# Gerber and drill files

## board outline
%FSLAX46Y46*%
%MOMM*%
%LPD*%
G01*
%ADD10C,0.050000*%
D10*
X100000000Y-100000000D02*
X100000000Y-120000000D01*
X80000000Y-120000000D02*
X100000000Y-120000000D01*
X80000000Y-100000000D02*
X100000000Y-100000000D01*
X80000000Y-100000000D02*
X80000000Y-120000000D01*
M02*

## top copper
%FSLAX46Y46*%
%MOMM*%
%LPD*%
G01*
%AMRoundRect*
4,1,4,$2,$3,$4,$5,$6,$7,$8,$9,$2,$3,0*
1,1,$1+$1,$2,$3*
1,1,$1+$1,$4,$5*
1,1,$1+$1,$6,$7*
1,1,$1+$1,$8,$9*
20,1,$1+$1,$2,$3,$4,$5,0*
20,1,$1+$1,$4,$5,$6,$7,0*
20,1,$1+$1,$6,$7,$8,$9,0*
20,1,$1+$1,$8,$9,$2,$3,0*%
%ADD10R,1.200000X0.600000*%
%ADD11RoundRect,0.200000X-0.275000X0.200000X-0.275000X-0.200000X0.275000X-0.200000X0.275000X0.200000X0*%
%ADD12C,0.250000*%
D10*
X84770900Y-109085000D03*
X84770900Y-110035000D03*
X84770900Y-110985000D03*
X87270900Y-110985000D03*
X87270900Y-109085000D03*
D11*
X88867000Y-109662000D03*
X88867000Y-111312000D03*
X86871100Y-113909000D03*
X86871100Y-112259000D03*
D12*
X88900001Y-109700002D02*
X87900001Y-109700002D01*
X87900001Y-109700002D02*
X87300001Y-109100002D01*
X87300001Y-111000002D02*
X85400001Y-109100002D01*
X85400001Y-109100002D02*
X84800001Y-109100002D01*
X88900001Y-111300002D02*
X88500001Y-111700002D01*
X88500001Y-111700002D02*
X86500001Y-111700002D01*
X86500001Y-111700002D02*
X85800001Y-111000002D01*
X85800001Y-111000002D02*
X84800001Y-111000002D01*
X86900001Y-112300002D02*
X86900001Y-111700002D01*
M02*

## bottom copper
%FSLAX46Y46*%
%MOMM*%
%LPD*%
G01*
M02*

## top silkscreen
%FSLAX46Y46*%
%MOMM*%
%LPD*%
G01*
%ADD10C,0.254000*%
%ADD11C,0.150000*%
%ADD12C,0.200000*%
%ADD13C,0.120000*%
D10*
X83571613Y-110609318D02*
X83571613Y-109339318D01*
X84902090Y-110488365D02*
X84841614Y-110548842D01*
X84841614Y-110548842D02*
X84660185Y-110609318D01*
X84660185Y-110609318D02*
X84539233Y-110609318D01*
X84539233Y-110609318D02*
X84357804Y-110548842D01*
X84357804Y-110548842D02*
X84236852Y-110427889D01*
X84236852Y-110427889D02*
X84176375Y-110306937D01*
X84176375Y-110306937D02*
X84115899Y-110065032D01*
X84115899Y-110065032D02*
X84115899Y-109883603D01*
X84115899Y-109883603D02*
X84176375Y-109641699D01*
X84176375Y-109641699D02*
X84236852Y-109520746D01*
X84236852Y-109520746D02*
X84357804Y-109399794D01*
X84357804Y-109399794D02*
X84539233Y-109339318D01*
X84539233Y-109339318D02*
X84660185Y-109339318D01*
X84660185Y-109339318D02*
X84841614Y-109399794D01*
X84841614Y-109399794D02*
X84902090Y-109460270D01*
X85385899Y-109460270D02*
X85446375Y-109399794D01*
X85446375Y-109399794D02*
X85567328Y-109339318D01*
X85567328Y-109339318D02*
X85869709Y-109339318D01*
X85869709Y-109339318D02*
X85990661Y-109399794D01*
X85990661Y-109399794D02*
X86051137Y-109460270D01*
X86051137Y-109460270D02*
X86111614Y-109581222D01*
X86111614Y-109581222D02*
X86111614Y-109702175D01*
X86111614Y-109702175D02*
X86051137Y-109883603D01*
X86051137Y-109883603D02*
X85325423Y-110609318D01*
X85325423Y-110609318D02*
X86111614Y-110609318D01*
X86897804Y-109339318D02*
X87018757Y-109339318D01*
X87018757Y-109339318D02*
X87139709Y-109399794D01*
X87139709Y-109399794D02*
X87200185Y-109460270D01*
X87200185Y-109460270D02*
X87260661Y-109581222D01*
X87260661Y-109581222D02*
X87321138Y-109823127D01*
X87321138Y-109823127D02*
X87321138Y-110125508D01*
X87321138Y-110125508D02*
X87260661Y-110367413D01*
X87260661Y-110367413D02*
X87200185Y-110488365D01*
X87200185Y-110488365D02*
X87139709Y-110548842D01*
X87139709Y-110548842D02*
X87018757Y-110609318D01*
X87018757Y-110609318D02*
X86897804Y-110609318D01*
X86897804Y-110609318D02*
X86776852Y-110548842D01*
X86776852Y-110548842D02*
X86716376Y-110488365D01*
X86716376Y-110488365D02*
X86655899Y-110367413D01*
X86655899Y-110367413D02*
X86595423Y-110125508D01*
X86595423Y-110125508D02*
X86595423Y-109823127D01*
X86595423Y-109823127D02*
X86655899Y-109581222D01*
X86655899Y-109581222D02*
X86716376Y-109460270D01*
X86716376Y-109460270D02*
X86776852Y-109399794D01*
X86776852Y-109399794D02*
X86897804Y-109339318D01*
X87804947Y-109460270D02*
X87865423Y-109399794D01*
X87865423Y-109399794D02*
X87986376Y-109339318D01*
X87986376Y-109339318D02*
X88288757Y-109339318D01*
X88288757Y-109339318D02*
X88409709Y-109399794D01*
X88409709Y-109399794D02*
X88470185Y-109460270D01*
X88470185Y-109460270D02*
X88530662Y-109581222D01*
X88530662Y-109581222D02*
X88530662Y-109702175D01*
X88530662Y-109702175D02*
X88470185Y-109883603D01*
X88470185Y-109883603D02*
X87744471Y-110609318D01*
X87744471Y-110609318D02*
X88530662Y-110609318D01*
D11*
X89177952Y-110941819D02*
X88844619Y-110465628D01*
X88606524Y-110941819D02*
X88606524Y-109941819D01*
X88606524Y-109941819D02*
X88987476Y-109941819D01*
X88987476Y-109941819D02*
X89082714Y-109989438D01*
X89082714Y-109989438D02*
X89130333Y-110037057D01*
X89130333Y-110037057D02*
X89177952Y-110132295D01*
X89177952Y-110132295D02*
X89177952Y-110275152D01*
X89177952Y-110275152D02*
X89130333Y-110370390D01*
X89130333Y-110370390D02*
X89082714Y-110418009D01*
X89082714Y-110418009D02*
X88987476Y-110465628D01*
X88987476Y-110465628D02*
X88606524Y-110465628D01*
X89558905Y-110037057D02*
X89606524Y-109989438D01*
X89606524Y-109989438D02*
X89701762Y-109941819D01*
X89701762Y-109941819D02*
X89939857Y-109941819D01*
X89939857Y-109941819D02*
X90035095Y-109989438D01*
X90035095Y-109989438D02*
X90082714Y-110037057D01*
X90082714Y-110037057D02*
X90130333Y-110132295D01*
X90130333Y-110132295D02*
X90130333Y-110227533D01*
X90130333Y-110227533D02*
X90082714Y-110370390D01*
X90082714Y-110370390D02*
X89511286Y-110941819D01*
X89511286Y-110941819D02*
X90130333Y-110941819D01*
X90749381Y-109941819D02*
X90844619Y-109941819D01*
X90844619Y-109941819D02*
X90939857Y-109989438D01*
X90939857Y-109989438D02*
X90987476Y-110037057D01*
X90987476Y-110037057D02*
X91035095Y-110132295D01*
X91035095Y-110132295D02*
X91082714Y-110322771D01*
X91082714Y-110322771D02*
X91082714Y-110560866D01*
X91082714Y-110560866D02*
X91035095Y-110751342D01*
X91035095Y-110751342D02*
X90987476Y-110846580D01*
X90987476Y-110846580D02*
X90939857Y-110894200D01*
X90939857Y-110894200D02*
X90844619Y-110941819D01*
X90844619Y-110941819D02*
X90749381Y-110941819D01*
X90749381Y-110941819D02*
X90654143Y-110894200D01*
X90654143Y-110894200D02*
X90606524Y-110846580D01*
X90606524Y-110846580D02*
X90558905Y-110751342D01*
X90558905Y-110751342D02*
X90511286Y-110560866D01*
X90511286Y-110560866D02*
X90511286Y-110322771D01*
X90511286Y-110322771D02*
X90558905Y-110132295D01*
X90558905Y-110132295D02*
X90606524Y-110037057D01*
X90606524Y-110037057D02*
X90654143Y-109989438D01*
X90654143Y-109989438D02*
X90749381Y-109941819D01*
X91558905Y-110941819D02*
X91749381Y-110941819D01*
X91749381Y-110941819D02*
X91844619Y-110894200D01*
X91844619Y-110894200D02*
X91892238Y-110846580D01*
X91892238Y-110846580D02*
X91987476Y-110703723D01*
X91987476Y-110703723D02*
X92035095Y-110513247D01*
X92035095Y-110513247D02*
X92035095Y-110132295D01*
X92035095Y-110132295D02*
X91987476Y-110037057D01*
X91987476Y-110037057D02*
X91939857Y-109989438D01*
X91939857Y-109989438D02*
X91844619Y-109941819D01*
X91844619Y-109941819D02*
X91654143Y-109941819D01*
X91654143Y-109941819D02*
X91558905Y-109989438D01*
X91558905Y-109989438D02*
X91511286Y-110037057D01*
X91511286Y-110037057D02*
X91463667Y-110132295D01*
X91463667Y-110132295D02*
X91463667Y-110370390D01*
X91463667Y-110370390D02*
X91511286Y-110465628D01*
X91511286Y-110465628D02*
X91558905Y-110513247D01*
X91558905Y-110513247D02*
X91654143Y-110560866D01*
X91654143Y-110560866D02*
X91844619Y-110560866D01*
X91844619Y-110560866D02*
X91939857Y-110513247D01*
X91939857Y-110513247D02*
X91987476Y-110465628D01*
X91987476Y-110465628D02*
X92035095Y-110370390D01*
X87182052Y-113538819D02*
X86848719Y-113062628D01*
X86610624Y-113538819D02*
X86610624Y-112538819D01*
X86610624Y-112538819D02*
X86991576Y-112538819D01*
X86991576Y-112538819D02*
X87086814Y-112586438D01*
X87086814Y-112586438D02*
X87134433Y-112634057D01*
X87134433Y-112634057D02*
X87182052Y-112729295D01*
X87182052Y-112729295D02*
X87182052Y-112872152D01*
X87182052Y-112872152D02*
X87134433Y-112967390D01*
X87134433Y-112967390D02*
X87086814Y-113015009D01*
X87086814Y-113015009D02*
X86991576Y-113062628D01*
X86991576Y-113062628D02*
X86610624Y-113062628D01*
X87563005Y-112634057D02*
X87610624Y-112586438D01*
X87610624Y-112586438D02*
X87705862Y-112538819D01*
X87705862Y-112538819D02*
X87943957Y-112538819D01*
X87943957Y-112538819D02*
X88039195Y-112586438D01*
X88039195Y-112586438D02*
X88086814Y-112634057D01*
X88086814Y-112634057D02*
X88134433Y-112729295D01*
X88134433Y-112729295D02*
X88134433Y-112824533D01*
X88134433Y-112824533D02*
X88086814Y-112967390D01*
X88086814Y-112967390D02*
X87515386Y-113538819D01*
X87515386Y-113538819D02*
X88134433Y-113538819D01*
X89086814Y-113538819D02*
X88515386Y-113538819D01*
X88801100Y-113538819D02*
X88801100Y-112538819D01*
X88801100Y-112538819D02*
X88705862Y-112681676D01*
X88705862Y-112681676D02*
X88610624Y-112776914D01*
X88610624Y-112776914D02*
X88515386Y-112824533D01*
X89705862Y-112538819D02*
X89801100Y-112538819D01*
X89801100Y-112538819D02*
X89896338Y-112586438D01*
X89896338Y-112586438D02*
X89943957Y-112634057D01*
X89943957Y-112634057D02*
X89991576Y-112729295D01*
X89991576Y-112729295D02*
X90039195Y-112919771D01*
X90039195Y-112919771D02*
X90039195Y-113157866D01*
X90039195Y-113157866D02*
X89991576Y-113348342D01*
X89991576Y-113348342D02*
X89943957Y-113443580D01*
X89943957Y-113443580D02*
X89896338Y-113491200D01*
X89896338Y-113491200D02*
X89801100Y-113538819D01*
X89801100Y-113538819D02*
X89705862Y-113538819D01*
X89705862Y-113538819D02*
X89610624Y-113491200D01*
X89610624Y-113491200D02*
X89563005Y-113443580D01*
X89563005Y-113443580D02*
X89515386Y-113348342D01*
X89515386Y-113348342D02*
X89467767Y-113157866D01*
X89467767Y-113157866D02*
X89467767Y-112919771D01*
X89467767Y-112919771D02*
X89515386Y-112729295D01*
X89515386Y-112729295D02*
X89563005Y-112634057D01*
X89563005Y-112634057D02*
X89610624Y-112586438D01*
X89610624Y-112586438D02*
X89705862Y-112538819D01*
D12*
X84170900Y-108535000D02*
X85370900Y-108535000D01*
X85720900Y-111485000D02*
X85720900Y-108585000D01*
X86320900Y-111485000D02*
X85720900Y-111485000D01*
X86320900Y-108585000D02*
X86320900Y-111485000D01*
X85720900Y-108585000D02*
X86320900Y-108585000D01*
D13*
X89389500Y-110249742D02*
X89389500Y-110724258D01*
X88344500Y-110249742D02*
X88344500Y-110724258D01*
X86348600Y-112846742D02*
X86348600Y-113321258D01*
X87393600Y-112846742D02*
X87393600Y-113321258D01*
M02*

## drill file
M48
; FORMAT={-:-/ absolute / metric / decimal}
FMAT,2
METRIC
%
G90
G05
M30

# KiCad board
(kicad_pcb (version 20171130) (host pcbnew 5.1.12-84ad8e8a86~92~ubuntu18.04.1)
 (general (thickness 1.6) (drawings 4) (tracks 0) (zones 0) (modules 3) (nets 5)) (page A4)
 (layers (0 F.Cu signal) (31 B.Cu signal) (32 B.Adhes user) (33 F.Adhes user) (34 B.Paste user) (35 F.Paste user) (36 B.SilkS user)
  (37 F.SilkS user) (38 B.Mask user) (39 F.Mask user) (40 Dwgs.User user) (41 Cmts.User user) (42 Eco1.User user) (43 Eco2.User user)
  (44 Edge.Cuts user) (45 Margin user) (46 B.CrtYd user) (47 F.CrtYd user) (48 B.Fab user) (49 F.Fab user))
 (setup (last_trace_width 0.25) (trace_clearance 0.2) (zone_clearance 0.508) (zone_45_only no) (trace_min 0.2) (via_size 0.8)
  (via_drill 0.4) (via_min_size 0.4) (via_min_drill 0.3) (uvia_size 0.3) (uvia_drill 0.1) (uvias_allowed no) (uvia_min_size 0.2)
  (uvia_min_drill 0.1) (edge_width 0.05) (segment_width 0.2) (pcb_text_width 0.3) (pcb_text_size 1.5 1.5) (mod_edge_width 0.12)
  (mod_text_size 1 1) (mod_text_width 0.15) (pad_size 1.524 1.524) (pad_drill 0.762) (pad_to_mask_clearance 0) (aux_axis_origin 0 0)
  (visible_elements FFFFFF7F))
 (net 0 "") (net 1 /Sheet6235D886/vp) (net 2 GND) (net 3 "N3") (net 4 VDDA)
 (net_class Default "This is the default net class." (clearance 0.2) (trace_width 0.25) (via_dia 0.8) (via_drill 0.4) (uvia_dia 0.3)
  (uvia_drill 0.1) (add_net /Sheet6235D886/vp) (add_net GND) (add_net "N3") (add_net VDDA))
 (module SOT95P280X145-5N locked (layer F.Cu) (at 86.020900 110.035000)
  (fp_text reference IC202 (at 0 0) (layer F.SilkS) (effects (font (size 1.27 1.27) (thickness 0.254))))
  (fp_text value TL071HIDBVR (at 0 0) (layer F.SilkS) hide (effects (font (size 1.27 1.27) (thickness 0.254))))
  (fp_line (start -1.85 -1.5) (end -0.65 -1.5) (layer F.SilkS) (width 0.2))
  (fp_line (start -0.3 1.45) (end -0.3 -1.45) (layer F.SilkS) (width 0.2))
  (fp_line (start 0.3 1.45) (end -0.3 1.45) (layer F.SilkS) (width 0.2))
  (fp_line (start 0.3 -1.45) (end 0.3 1.45) (layer F.SilkS) (width 0.2))
  (fp_line (start -0.3 -1.45) (end 0.3 -1.45) (layer F.SilkS) (width 0.2))
  (pad 1 smd rect (at -1.25 -0.95 90.000000) (size 0.6 1.2) (layers F.Cu F.Mask F.Paste) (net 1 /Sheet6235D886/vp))
  (pad 2 smd rect (at -1.25 0 90.000000) (size 0.6 1.2) (layers F.Cu F.Mask F.Paste) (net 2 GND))
  (pad 3 smd rect (at -1.25 0.95 90.000000) (size 0.6 1.2) (layers F.Cu F.Mask F.Paste) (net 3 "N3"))
  (pad 4 smd rect (at 1.25 0.95 90.000000) (size 0.6 1.2) (layers F.Cu F.Mask F.Paste) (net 1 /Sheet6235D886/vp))
  (pad 5 smd rect (at 1.25 -0.95 90.000000) (size 0.6 1.2) (layers F.Cu F.Mask F.Paste) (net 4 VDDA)))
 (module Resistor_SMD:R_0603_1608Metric (layer F.Cu) (at 88.867000 110.487000 270.000000)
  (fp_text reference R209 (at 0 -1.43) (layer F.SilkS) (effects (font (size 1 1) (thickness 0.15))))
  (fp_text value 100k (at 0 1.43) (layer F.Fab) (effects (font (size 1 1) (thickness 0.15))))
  (fp_line (start -0.237258 -0.5225) (end 0.237258 -0.5225) (layer F.SilkS) (width 0.12))
  (fp_line (start -0.237258 0.5225) (end 0.237258 0.5225) (layer F.SilkS) (width 0.12))
  (pad 1 smd roundrect (at -0.825 0 270.000000) (size 0.8 0.95) (layers F.Cu F.Mask F.Paste) (roundrect_rratio 0.25) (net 4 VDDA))
  (pad 2 smd roundrect (at 0.825 0 270.000000) (size 0.8 0.95) (layers F.Cu F.Mask F.Paste) (roundrect_rratio 0.25) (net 3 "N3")))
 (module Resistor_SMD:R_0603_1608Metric (layer F.Cu) (at 86.871100 113.084000 270.000000)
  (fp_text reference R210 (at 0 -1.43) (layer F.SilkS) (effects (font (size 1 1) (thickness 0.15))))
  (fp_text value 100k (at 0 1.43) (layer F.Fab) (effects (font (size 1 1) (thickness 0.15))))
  (fp_line (start -0.237258 0.5225) (end 0.237258 0.5225) (layer F.SilkS) (width 0.12))
  (fp_line (start -0.237258 -0.5225) (end 0.237258 -0.5225) (layer F.SilkS) (width 0.12))
  (pad 2 smd roundrect (at 0.825 0 270.000000) (size 0.8 0.95) (layers F.Cu F.Mask F.Paste) (roundrect_rratio 0.25) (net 2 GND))
  (pad 1 smd roundrect (at -0.825 0 270.000000) (size 0.8 0.95) (layers F.Cu F.Mask F.Paste) (roundrect_rratio 0.25) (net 3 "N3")))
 (gr_line (start 100 100) (end 100 120) (layer Edge.Cuts) (width 0.05))
 (gr_line (start 80 120) (end 100 120) (layer Edge.Cuts) (width 0.05))
 (gr_line (start 80 100) (end 100 100) (layer Edge.Cuts) (width 0.05))
 (gr_line (start 80 100) (end 80 120) (layer Edge.Cuts) (width 0.05))
 (segment (start 88.900001 109.700002) (end 87.900001 109.700002) (width 0.250000) (layer F.Cu) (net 4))
 (segment (start 87.900001 109.700002) (end 87.300001 109.100002) (width 0.250000) (layer F.Cu) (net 4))
 (segment (start 87.300001 111.000002) (end 85.400001 109.100002) (width 0.250000) (layer F.Cu) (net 1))
 (segment (start 85.400001 109.100002) (end 84.800001 109.100002) (width 0.250000) (layer F.Cu) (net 1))
 (segment (start 88.900001 111.300002) (end 88.500001 111.700002) (width 0.250000) (layer F.Cu) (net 3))
 (segment (start 88.500001 111.700002) (end 86.500001 111.700002) (width 0.250000) (layer F.Cu) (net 3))
 (segment (start 86.500001 111.700002) (end 85.800001 111.000002) (width 0.250000) (layer F.Cu) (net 3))
 (segment (start 85.800001 111.000002) (end 84.800001 111.000002) (width 0.250000) (layer F.Cu) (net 3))
 (segment (start 86.900001 112.300002) (end 86.900001 111.700002) (width 0.250000) (layer F.Cu) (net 3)))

